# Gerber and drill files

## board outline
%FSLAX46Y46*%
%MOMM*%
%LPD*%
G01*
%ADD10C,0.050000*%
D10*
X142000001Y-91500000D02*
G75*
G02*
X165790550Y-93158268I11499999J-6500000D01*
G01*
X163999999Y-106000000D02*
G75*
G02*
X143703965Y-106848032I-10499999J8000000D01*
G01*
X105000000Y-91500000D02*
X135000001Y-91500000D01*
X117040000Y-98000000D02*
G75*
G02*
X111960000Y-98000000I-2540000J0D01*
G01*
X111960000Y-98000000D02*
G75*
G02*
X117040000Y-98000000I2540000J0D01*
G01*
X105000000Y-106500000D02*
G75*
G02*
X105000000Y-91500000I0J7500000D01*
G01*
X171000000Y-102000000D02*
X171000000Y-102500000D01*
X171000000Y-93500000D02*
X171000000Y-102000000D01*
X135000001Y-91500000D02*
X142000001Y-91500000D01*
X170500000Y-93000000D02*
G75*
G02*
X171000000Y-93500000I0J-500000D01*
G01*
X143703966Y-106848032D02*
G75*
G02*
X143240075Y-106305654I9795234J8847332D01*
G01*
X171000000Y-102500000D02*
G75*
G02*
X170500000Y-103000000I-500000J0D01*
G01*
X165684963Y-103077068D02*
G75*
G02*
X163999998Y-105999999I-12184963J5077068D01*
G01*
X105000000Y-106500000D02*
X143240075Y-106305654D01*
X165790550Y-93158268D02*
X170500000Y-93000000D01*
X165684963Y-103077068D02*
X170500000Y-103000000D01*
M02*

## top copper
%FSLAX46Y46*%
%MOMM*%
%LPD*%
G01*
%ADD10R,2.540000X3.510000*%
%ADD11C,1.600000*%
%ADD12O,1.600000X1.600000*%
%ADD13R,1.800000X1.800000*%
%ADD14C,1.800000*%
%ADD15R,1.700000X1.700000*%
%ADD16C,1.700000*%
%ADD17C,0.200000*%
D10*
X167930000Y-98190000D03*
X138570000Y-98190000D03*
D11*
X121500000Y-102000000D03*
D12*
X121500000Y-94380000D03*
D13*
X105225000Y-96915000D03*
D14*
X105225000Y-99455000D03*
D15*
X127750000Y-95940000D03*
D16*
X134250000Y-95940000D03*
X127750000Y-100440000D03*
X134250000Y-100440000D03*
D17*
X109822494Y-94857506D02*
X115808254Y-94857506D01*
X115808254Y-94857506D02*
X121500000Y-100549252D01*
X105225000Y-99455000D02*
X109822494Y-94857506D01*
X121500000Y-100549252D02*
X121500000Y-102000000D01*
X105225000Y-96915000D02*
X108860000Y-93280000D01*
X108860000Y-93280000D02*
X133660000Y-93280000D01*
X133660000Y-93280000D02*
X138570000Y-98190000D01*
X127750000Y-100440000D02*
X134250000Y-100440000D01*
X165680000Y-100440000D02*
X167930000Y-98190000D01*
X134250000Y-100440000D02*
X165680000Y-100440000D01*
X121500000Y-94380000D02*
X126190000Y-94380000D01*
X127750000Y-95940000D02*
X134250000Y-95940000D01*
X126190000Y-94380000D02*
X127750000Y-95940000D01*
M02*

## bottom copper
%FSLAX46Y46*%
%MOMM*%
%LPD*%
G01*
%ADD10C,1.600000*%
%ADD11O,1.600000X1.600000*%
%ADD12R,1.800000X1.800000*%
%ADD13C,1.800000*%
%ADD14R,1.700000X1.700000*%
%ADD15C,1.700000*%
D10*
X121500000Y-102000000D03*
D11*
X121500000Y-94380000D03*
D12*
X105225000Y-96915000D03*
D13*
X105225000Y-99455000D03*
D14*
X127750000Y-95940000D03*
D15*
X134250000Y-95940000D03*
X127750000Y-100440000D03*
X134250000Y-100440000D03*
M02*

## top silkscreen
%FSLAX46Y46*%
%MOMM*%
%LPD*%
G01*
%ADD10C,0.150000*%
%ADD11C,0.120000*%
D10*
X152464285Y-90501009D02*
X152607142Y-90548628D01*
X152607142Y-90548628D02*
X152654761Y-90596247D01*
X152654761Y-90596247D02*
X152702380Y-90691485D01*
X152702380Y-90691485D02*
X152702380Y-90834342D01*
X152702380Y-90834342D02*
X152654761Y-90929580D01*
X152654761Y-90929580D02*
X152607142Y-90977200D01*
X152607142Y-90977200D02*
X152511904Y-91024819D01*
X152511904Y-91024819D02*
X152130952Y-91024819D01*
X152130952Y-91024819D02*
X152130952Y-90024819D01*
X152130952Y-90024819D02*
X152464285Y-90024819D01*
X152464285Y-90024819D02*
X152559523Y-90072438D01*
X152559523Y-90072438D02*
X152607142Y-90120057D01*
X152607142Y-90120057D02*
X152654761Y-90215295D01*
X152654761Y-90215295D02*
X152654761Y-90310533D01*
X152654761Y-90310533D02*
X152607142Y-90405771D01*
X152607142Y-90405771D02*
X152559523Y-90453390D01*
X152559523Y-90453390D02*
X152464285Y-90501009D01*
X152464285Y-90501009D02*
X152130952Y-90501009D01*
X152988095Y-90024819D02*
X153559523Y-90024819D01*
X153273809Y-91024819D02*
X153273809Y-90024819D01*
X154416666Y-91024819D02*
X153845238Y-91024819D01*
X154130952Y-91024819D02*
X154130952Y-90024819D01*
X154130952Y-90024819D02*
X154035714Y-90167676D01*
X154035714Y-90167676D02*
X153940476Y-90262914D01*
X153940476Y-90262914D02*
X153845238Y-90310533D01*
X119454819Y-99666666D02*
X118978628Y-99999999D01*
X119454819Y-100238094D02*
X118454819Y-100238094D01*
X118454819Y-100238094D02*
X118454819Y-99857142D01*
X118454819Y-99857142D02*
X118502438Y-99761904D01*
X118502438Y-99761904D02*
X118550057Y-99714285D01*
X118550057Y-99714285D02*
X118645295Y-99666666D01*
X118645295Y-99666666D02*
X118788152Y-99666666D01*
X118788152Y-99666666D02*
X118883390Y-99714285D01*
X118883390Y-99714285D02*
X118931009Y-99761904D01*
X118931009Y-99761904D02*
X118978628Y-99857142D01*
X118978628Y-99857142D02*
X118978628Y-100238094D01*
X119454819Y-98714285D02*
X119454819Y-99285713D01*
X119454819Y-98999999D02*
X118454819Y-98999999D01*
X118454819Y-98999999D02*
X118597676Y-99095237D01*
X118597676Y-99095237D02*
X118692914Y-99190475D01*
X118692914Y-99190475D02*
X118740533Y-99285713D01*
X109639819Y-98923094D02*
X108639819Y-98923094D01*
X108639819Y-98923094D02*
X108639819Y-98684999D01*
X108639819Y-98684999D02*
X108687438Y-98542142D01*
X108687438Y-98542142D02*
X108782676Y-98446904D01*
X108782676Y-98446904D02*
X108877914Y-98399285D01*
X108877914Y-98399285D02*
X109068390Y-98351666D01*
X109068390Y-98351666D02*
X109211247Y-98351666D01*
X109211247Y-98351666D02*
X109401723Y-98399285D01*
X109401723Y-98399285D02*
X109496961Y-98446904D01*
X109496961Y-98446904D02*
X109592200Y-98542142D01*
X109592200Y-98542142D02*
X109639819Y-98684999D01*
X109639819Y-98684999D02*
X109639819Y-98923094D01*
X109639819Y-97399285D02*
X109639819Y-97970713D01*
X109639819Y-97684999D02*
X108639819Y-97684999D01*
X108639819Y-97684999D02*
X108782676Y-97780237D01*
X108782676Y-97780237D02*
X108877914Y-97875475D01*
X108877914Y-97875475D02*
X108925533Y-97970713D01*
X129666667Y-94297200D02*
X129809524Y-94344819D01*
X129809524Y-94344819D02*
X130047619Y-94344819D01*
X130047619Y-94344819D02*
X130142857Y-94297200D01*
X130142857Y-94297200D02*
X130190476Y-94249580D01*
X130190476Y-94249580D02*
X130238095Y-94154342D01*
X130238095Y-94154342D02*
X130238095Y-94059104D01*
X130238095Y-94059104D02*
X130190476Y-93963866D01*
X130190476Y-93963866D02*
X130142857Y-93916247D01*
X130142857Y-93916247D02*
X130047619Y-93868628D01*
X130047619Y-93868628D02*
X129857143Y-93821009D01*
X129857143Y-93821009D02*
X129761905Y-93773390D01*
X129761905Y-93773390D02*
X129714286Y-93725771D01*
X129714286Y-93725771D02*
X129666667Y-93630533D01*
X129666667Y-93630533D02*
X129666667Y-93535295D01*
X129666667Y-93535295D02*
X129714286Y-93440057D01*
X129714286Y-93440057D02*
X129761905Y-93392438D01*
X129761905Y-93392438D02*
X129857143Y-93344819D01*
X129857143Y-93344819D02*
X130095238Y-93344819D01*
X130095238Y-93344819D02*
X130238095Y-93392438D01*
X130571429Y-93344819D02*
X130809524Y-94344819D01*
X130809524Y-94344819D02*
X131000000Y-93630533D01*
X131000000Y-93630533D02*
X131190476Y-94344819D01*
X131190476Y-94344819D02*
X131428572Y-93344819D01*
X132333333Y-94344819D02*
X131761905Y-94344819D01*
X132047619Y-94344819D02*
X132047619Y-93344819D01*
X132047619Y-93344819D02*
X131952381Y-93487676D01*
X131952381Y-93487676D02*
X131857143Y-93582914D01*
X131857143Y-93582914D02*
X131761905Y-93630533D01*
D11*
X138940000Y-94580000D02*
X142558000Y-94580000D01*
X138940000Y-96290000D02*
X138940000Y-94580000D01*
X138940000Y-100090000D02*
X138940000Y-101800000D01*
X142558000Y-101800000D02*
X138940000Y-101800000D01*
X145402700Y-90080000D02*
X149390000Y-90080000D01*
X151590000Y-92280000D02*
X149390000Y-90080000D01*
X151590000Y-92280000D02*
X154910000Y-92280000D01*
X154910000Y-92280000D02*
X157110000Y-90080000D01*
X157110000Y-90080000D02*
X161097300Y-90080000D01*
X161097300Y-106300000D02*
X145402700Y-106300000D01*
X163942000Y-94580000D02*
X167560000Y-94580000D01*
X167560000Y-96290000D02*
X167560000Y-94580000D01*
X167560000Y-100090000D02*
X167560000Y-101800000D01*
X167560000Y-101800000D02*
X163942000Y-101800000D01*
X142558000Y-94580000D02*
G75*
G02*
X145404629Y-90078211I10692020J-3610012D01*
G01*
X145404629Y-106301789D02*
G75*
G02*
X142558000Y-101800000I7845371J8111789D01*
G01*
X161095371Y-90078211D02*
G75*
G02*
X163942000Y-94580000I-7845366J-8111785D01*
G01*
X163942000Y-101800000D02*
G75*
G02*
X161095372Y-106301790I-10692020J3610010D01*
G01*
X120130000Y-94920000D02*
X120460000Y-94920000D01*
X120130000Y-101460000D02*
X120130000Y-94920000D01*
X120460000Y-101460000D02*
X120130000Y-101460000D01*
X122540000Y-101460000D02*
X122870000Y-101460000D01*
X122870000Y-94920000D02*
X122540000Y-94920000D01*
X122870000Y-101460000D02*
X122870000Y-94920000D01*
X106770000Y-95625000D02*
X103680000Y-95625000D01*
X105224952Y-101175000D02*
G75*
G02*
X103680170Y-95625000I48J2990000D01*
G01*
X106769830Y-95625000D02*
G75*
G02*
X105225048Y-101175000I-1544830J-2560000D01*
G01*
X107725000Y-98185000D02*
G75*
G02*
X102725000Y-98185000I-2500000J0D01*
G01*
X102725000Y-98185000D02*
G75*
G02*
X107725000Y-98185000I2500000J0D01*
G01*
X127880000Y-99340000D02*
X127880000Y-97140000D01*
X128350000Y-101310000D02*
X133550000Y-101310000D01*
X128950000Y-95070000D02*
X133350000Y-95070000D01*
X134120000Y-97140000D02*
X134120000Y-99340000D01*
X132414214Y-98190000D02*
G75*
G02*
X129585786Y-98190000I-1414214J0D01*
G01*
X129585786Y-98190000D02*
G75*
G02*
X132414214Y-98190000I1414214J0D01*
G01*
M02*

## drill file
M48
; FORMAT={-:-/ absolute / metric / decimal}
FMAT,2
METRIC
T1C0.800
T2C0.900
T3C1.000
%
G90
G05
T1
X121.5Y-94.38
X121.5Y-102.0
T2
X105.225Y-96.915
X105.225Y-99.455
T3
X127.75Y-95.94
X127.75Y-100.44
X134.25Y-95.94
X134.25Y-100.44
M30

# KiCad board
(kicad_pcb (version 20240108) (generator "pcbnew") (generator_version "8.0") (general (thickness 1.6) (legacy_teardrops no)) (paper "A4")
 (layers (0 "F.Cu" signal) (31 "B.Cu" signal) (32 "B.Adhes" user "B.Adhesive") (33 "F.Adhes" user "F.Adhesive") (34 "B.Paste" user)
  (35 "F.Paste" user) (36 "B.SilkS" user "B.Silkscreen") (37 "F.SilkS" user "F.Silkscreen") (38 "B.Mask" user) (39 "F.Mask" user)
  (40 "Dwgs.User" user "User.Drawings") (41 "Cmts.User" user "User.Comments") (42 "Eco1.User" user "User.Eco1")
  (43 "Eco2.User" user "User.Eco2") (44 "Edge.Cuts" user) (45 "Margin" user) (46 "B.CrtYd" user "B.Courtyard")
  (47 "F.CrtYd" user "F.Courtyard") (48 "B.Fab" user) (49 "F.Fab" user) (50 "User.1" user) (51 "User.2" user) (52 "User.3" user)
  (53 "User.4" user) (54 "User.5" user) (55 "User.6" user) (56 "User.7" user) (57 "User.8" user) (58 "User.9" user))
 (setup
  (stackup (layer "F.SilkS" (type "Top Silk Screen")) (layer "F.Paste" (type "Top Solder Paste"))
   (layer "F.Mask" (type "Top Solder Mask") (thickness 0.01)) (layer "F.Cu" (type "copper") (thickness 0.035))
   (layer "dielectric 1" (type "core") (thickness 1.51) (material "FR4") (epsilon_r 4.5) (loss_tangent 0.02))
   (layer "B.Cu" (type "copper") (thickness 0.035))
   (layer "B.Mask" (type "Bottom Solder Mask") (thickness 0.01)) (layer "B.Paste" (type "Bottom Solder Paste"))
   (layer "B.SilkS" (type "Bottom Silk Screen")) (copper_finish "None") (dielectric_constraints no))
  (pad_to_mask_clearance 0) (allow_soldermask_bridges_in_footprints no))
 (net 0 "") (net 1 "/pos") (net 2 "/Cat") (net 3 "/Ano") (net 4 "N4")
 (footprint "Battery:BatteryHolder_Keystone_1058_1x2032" (layer "F.Cu") (at 153.25 98.19 180)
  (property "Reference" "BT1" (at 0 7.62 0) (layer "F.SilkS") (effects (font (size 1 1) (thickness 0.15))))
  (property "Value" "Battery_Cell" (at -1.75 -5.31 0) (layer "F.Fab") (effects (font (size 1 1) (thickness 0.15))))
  (fp_line (start 14.31 3.61) (end 10.692 3.61) (stroke (width 0.12) (type solid)) (layer "F.SilkS"))
  (fp_line (start 14.31 1.9) (end 14.31 3.61) (stroke (width 0.12) (type solid)) (layer "F.SilkS"))
  (fp_line (start 14.31 -1.9) (end 14.31 -3.61) (stroke (width 0.12) (type solid)) (layer "F.SilkS"))
  (fp_line (start 10.692 -3.61) (end 14.31 -3.61) (stroke (width 0.12) (type solid)) (layer "F.SilkS"))
  (fp_line (start 7.8473 8.11) (end 3.86 8.11) (stroke (width 0.12) (type solid)) (layer "F.SilkS"))
  (fp_line (start 1.66 5.91) (end 3.86 8.11) (stroke (width 0.12) (type solid)) (layer "F.SilkS"))
  (fp_line (start 1.66 5.91) (end -1.66 5.91) (stroke (width 0.12) (type solid)) (layer "F.SilkS"))
  (fp_line (start -1.66 5.91) (end -3.86 8.11) (stroke (width 0.12) (type solid)) (layer "F.SilkS"))
  (fp_line (start -3.86 8.11) (end -7.8473 8.11) (stroke (width 0.12) (type solid)) (layer "F.SilkS"))
  (fp_line (start -7.8473 -8.11) (end 7.8473 -8.11) (stroke (width 0.12) (type solid)) (layer "F.SilkS"))
  (fp_line (start -10.692 3.61) (end -14.31 3.61) (stroke (width 0.12) (type solid)) (layer "F.SilkS"))
  (fp_line (start -14.31 1.9) (end -14.31 3.61) (stroke (width 0.12) (type solid)) (layer "F.SilkS"))
  (fp_line (start -14.31 -1.9) (end -14.31 -3.61) (stroke (width 0.12) (type solid)) (layer "F.SilkS"))
  (fp_line (start -14.31 -3.61) (end -10.692 -3.61) (stroke (width 0.12) (type solid)) (layer "F.SilkS"))
  (fp_arc (start 10.692 3.61) (mid 9.538084 6.031244) (end 7.845371 8.111789) (stroke (width 0.12) (type solid)) (layer "F.SilkS"))
  (fp_arc (start 7.845371 -8.111789) (mid 9.538085 -6.031244) (end 10.692 -3.61) (stroke (width 0.12) (type solid)) (layer "F.SilkS"))
  (fp_arc (start -7.845371 8.111789) (mid -9.538085 6.031244) (end -10.692 3.61) (stroke (width 0.12) (type solid)) (layer "F.SilkS"))
  (fp_arc (start -10.692 -3.61) (mid -9.538084 -6.031244) (end -7.845371 -8.111789) (stroke (width 0.12) (type solid)) (layer "F.SilkS"))
  (pad "1" smd rect (at -14.68 0 180) (size 2.54 3.51) (layers "F.Cu" "F.Paste" "F.Mask") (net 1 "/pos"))
  (pad "2" smd rect (at 14.68 0 180) (size 2.54 3.51) (layers "F.Cu" "F.Paste" "F.Mask") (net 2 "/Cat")))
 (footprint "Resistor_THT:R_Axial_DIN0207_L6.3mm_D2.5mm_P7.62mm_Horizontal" (layer "F.Cu") (at 121.5 102 90)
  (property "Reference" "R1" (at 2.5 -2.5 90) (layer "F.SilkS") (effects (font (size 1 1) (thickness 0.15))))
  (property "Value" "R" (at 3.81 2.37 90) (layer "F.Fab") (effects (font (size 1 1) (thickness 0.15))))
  (fp_line (start 7.08 -1.37) (end 7.08 -1.04) (stroke (width 0.12) (type solid)) (layer "F.SilkS"))
  (fp_line (start 0.54 -1.37) (end 7.08 -1.37) (stroke (width 0.12) (type solid)) (layer "F.SilkS"))
  (fp_line (start 0.54 -1.04) (end 0.54 -1.37) (stroke (width 0.12) (type solid)) (layer "F.SilkS"))
  (fp_line (start 0.54 1.04) (end 0.54 1.37) (stroke (width 0.12) (type solid)) (layer "F.SilkS"))
  (fp_line (start 7.08 1.37) (end 7.08 1.04) (stroke (width 0.12) (type solid)) (layer "F.SilkS"))
  (fp_line (start 0.54 1.37) (end 7.08 1.37) (stroke (width 0.12) (type solid)) (layer "F.SilkS"))
  (pad "1" thru_hole circle (at 0 0 90) (size 1.6 1.6) (drill 0.8) (layers "*.Cu" "*.Mask") (remove_unused_layers no) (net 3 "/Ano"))
  (pad "2" thru_hole oval (at 7.62 0 90) (size 1.6 1.6) (drill 0.8) (layers "*.Cu" "*.Mask") (remove_unused_layers no) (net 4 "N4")))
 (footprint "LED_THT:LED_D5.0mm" (layer "F.Cu") (at 105.225 96.915 -90)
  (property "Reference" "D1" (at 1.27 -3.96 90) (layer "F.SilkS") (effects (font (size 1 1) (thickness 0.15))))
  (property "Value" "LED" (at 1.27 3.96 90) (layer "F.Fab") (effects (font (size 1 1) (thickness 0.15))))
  (fp_line (start -1.29 -1.545) (end -1.29 1.545) (stroke (width 0.12) (type solid)) (layer "F.SilkS"))
  (fp_arc (start 4.26 0.000048) (mid 2.071756 2.880501) (end -1.29 1.54483) (stroke (width 0.12) (type solid)) (layer "F.SilkS"))
  (fp_arc (start -1.29 -1.54483) (mid 2.071756 -2.880501) (end 4.26 -0.000048) (stroke (width 0.12) (type solid)) (layer "F.SilkS"))
  (fp_circle (center 1.27 0) (end 3.77 0) (stroke (width 0.12) (type solid)) (fill none) (layer "F.SilkS"))
  (pad "1" thru_hole rect (at 0 0 270) (size 1.8 1.8) (drill 0.9) (layers "*.Cu" "*.Mask") (remove_unused_layers no) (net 2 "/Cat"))
  (pad "2" thru_hole circle (at 2.54 0 270) (size 1.8 1.8) (drill 0.9) (layers "*.Cu" "*.Mask") (remove_unused_layers no) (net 3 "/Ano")))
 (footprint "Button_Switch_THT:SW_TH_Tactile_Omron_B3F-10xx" (layer "F.Cu") (at 127.75 95.94)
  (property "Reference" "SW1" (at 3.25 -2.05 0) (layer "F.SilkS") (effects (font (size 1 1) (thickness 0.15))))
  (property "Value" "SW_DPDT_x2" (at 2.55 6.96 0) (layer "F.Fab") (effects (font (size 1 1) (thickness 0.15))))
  (fp_line (start 0.13 3.4) (end 0.13 1.2) (stroke (width 0.12) (type solid)) (layer "F.SilkS"))
  (fp_line (start 0.6 5.37) (end 5.8 5.37) (stroke (width 0.12) (type solid)) (layer "F.SilkS"))
  (fp_line (start 1.2 -0.87) (end 5.6 -0.87) (stroke (width 0.12) (type solid)) (layer "F.SilkS"))
  (fp_line (start 6.37 1.2) (end 6.37 3.4) (stroke (width 0.12) (type solid)) (layer "F.SilkS"))
  (fp_circle (center 3.25 2.25) (end 4.25 3.25) (stroke (width 0.12) (type solid)) (fill none) (layer "F.SilkS"))
  (pad "1" thru_hole rect (at 0 0) (size 1.7 1.7) (drill 1) (layers "*.Cu" "*.Mask") (remove_unused_layers no) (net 4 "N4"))
  (pad "1" thru_hole circle (at 6.5 0) (size 1.7 1.7) (drill 1) (layers "*.Cu" "*.Mask") (remove_unused_layers no) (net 4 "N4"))
  (pad "2" thru_hole circle (at 0 4.5) (size 1.7 1.7) (drill 1) (layers "*.Cu" "*.Mask") (remove_unused_layers no) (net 1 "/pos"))
  (pad "2" thru_hole circle (at 6.5 4.5) (size 1.7 1.7) (drill 1) (layers "*.Cu" "*.Mask") (remove_unused_layers no) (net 1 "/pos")))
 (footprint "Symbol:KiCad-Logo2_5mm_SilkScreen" (layer "B.Cu") (at 154.25 97.3 180)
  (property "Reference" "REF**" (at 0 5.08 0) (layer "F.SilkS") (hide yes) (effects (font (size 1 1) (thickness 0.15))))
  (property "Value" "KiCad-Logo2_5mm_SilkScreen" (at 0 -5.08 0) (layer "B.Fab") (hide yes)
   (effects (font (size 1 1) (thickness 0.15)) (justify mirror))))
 (gr_arc (start 142.000001 91.5) (mid 154.418535 84.822129) (end 165.79055 93.158268) (locked yes) (stroke (width 0.05) (type default))
  (layer "Edge.Cuts"))
 (gr_arc (start 163.999999 106) (mid 154.051073 111.18887) (end 143.703965 106.848032) (locked yes) (stroke (width 0.05) (type default))
  (layer "Edge.Cuts"))
 (gr_line (start 105 91.5) (end 135.000001 91.5) (locked yes) (stroke (width 0.05) (type default)) (layer "Edge.Cuts"))
 (gr_circle (center 114.5 98) (end 114.5 100.54) (stroke (width 0.05) (type default)) (fill none) (layer "Edge.Cuts"))
 (gr_arc (start 105 106.5) (mid 97.5 99) (end 105 91.5) (locked yes) (stroke (width 0.05) (type default)) (layer "Edge.Cuts"))
 (gr_line (start 171 102) (end 171 102.5) (locked yes) (stroke (width 0.05) (type default)) (layer "Edge.Cuts"))
 (gr_line (start 171 93.5) (end 171 102) (locked yes) (stroke (width 0.05) (type default)) (layer "Edge.Cuts"))
 (gr_line (start 135.000001 91.5) (end 142.000001 91.5) (locked yes) (stroke (width 0.05) (type default)) (layer "Edge.Cuts"))
 (gr_arc (start 170.5 93) (mid 170.853553 93.146447) (end 171 93.5) (locked yes) (stroke (width 0.05) (type default)) (layer "Edge.Cuts"))
 (gr_arc (start 143.703966 106.848032) (mid 143.468354 106.579979) (end 143.240075 106.305654) (locked yes)
  (stroke (width 0.05) (type default)) (layer "Edge.Cuts"))
 (gr_arc (start 171 102.5) (mid 170.853553 102.853553) (end 170.5 103) (locked yes) (stroke (width 0.05) (type default)) (layer "Edge.Cuts"))
 (gr_arc (start 165.684963 103.077068) (mid 164.936247 104.592587) (end 163.999998 105.999999) (locked yes)
  (stroke (width 0.05) (type default)) (layer "Edge.Cuts"))
 (gr_line (start 105 106.5) (end 143.240075 106.305654) (locked yes) (stroke (width 0.05) (type default)) (layer "Edge.Cuts"))
 (gr_line (start 165.79055 93.158268) (end 170.5 93) (locked yes) (stroke (width 0.05) (type default)) (layer "Edge.Cuts"))
 (gr_line (start 165.684963 103.077068) (end 170.5 103) (locked yes) (stroke (width 0.05) (type default)) (layer "Edge.Cuts"))
 (segment (start 109.822494 94.857506) (end 115.808254 94.857506) (width 0.2) (layer "F.Cu") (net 3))
 (segment (start 115.808254 94.857506) (end 121.5 100.549252) (width 0.2) (layer "F.Cu") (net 3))
 (segment (start 105.225 99.455) (end 109.822494 94.857506) (width 0.2) (layer "F.Cu") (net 3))
 (segment (start 121.5 100.549252) (end 121.5 102) (width 0.2) (layer "F.Cu") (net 3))
 (segment (start 105.225 96.915) (end 108.86 93.28) (width 0.2) (layer "F.Cu") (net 2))
 (segment (start 108.86 93.28) (end 133.66 93.28) (width 0.2) (layer "F.Cu") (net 2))
 (segment (start 133.66 93.28) (end 138.57 98.19) (width 0.2) (layer "F.Cu") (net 2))
 (segment (start 127.75 100.44) (end 134.25 100.44) (width 0.2) (layer "F.Cu") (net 1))
 (segment (start 165.68 100.44) (end 167.93 98.19) (width 0.2) (layer "F.Cu") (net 1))
 (segment (start 134.25 100.44) (end 165.68 100.44) (width 0.2) (layer "F.Cu") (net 1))
 (segment (start 121.5 94.38) (end 126.19 94.38) (width 0.2) (layer "F.Cu") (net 4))
 (segment (start 127.75 95.94) (end 134.25 95.94) (width 0.2) (layer "F.Cu") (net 4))
 (segment (start 126.19 94.38) (end 127.75 95.94) (width 0.2) (layer "F.Cu") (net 4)))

